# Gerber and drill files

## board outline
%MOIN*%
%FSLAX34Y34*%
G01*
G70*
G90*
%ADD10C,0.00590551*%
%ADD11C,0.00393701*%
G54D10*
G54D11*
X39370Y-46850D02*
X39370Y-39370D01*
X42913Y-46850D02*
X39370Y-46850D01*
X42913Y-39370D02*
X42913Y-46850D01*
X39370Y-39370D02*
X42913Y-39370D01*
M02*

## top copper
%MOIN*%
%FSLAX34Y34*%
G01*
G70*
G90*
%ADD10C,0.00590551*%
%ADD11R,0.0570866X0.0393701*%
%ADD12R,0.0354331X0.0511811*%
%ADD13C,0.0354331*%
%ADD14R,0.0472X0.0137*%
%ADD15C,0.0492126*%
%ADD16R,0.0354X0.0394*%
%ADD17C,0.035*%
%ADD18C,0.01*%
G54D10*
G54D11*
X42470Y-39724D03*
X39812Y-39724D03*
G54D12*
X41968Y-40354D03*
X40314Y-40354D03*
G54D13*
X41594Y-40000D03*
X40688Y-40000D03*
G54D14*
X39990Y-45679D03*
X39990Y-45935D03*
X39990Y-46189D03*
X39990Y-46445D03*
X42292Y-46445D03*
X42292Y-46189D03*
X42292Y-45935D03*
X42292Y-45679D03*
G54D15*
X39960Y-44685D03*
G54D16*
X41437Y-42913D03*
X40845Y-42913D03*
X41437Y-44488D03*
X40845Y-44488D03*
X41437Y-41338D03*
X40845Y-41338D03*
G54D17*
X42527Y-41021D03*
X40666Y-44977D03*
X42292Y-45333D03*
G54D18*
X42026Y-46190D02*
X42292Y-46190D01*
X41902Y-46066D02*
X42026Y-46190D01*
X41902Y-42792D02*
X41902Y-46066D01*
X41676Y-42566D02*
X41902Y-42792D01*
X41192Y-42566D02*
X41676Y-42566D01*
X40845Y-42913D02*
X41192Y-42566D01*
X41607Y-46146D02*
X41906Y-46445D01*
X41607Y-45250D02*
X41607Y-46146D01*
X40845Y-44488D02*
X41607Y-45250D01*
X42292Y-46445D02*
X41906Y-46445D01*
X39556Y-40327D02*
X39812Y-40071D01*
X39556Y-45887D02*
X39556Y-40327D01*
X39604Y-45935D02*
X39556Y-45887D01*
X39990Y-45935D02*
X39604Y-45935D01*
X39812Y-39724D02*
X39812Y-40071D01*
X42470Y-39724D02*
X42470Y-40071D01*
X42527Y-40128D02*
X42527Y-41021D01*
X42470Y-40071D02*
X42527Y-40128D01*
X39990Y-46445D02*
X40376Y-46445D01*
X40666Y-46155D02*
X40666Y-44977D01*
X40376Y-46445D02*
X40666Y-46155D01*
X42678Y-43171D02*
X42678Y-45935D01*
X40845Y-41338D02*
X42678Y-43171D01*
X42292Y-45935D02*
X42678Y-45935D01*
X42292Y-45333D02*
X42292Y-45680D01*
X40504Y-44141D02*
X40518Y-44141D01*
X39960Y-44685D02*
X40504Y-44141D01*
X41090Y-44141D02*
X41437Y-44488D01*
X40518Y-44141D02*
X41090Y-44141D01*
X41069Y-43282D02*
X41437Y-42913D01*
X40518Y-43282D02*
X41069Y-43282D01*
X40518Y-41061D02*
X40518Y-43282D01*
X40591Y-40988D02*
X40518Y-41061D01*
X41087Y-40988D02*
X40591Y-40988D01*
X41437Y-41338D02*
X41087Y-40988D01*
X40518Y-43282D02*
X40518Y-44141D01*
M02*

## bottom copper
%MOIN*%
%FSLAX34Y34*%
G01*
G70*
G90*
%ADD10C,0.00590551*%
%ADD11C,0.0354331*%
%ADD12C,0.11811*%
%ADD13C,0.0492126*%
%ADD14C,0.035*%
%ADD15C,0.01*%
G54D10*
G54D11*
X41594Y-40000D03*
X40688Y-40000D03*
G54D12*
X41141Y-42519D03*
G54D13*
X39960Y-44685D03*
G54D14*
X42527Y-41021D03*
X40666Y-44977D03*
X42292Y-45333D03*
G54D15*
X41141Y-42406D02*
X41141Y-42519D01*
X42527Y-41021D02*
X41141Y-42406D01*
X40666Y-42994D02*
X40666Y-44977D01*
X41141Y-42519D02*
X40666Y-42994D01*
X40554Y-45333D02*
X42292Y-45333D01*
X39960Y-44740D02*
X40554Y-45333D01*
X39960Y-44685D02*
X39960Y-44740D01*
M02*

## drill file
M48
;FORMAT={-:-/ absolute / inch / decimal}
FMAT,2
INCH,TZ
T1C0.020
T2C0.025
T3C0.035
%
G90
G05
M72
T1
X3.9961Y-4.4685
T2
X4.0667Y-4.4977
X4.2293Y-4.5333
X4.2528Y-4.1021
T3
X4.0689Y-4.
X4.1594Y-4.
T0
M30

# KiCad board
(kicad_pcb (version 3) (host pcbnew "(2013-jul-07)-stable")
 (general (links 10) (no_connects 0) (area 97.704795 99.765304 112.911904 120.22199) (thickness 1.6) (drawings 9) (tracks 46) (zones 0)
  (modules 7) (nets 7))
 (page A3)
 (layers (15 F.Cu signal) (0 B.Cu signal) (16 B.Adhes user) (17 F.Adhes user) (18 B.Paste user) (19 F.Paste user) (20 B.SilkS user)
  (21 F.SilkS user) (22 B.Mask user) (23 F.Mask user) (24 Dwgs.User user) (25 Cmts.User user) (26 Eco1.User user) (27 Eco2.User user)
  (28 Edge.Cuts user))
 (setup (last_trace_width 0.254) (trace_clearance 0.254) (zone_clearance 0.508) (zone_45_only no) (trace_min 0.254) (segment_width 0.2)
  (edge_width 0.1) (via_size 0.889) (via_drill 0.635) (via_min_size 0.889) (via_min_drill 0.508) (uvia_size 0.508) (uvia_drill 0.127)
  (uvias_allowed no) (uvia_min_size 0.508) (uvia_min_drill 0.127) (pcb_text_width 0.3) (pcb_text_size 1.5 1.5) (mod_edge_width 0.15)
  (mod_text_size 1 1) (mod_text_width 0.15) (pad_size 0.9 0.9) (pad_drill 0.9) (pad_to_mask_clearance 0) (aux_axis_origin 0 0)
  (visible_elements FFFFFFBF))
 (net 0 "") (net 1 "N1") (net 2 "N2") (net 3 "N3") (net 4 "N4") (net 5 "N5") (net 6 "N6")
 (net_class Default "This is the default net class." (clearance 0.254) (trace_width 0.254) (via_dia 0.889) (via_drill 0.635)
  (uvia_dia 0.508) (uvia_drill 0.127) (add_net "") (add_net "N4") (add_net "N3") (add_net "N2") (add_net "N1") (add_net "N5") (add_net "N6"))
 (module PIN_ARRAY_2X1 (layer F.Cu) (at 104.5 101.6 180)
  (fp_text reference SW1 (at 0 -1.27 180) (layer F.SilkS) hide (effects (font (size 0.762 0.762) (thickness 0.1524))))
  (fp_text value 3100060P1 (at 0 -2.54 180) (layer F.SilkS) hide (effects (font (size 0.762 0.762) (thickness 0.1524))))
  (pad 1 smd rect (at -3.375 0.7 180) (size 1.45 1) (layers F.Cu F.Paste F.Mask) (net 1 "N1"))
  (pad 2 smd rect (at 3.375 0.7 180) (size 1.45 1) (layers F.Cu F.Paste F.Mask) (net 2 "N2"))
  (pad 3 smd rect (at -2.1 -0.9 180) (size 0.9 1.3) (layers F.Cu F.Paste F.Mask))
  (pad 4 smd rect (at 2.1 -0.9 180) (size 0.9 1.3) (layers F.Cu F.Paste F.Mask))
  (pad "" thru_hole circle (at -1.15 0 180) (size 0.9 0.9) (drill 0.9) (layers *.Cu *.Mask F.SilkS))
  (pad "" thru_hole circle (at 1.15 0 180) (size 0.9 0.9) (drill 0.9) (layers *.Cu *.Mask F.SilkS)))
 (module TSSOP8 (layer F.Cu) (at 104.5 117)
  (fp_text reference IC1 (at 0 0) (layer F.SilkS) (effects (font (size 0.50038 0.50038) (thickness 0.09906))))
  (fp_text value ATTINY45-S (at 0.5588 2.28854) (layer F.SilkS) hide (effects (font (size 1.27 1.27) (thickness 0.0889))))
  (pad 1 smd rect (at -2.92354 -0.97282) (size 1.19888 0.34798) (layers F.Cu F.Paste F.Mask))
  (pad 2 smd rect (at -2.92354 -0.32258) (size 1.19888 0.34798) (layers F.Cu F.Paste F.Mask) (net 2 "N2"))
  (pad 3 smd rect (at -2.92354 0.32258) (size 1.19888 0.34798) (layers F.Cu F.Paste F.Mask))
  (pad 4 smd rect (at -2.92354 0.97282) (size 1.19888 0.34798) (layers F.Cu F.Paste F.Mask) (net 1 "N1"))
  (pad 5 smd rect (at 2.92354 0.97282) (size 1.19888 0.34798) (layers F.Cu F.Paste F.Mask) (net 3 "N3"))
  (pad 6 smd rect (at 2.92354 0.32258) (size 1.19888 0.34798) (layers F.Cu F.Paste F.Mask) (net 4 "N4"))
  (pad 7 smd rect (at 2.92354 -0.32258) (size 1.19888 0.34798) (layers F.Cu F.Paste F.Mask) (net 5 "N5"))
  (pad 8 smd rect (at 2.92354 -0.97282) (size 1.19888 0.34798) (layers F.Cu F.Paste F.Mask) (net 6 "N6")))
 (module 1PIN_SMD (layer B.Cu) (at 104.5 108)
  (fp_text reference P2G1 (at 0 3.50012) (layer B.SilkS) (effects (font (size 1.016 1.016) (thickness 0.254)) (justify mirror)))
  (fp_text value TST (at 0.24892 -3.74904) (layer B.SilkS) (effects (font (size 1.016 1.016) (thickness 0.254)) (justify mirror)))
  (pad 1 smd circle (at 0 0) (size 3 3) (layers B.Cu B.Paste B.SilkS B.Mask) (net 1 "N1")))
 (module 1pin (layer F.Cu) (at 101.5 113.5)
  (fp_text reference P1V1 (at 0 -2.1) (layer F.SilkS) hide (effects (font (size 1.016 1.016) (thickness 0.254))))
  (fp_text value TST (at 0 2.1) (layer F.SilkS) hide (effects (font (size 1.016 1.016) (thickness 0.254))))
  (pad 1 thru_hole circle (at 0 0) (size 1.25 1.25) (drill 0.5) (layers *.Cu *.Mask F.SilkS) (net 6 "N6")))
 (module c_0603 (layer F.Cu) (at 104.5 109)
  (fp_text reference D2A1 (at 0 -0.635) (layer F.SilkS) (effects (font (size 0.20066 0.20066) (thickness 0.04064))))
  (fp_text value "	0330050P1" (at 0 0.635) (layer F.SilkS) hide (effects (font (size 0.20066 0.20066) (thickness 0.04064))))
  (pad 1 smd rect (at 0.75184 0) (size 0.89916 1.00076) (layers F.Cu F.Paste F.Mask) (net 6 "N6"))
  (pad 2 smd rect (at -0.75184 0) (size 0.89916 1.00076) (layers F.Cu F.Paste F.Mask) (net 4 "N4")))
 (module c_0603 (layer F.Cu) (at 104.5 113)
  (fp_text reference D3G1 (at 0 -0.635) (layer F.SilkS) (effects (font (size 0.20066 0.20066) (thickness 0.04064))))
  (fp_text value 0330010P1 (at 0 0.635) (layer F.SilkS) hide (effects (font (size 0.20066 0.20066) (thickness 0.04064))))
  (pad 1 smd rect (at 0.75184 0) (size 0.89916 1.00076) (layers F.Cu F.Paste F.Mask) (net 6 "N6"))
  (pad 2 smd rect (at -0.75184 0) (size 0.89916 1.00076) (layers F.Cu F.Paste F.Mask) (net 3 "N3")))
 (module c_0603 (layer F.Cu) (at 104.5 105)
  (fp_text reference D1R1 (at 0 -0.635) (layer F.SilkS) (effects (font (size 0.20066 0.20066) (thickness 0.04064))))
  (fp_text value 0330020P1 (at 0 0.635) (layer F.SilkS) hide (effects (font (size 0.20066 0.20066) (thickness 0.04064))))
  (pad 1 smd rect (at 0.75184 0) (size 0.89916 1.00076) (layers F.Cu F.Paste F.Mask) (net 6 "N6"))
  (pad 2 smd rect (at -0.75184 0) (size 0.89916 1.00076) (layers F.Cu F.Paste F.Mask) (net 5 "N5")))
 (gr_line (start 100 119) (end 100 100) (angle 90) (layer Edge.Cuts) (width 0.1))
 (gr_line (start 109 119) (end 100 119) (angle 90) (layer Edge.Cuts) (width 0.1))
 (gr_line (start 109 100) (end 109 119) (angle 90) (layer Edge.Cuts) (width 0.1))
 (gr_line (start 100 100) (end 109 100) (angle 90) (layer Edge.Cuts) (width 0.1))
 (segment (start 106.7483 117.3226) (end 107.4235 117.3226) (width 0.254) (layer F.Cu) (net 4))
 (segment (start 106.4335 117.0078) (end 106.7483 117.3226) (width 0.254) (layer F.Cu) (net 4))
 (segment (start 106.4335 108.6924) (end 106.4335 117.0078) (width 0.254) (layer F.Cu) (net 4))
 (segment (start 105.8593 108.1182) (end 106.4335 108.6924) (width 0.254) (layer F.Cu) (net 4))
 (segment (start 104.63 108.1182) (end 105.8593 108.1182) (width 0.254) (layer F.Cu) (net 4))
 (segment (start 103.7482 109) (end 104.63 108.1182) (width 0.254) (layer F.Cu) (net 4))
 (segment (start 105.6833 117.2133) (end 106.4428 117.9728) (width 0.254) (layer F.Cu) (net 3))
 (segment (start 105.6833 114.9351) (end 105.6833 117.2133) (width 0.254) (layer F.Cu) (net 3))
 (segment (start 103.7482 113) (end 105.6833 114.9351) (width 0.254) (layer F.Cu) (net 3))
 (segment (start 107.4235 117.9728) (end 106.4428 117.9728) (width 0.254) (layer F.Cu) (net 3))
 (segment (start 100.4738 102.4325) (end 101.125 101.7813) (width 0.254) (layer F.Cu) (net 2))
 (segment (start 100.4738 116.5554) (end 100.4738 102.4325) (width 0.254) (layer F.Cu) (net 2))
 (segment (start 100.5958 116.6774) (end 100.4738 116.5554) (width 0.254) (layer F.Cu) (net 2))
 (segment (start 101.5765 116.6774) (end 100.5958 116.6774) (width 0.254) (layer F.Cu) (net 2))
 (segment (start 101.125 100.9) (end 101.125 101.7813) (width 0.254) (layer F.Cu) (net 2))
 (via (at 108.02 104.1936) (size 0.889) (layers F.Cu B.Cu) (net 1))
 (via (at 103.294 114.2421) (size 0.889) (layers F.Cu B.Cu) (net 1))
 (segment (start 107.875 100.9) (end 107.875 101.7813) (width 0.254) (layer F.Cu) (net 1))
 (segment (start 108.02 101.9263) (end 108.02 104.1936) (width 0.254) (layer F.Cu) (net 1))
 (segment (start 107.875 101.7813) (end 108.02 101.9263) (width 0.254) (layer F.Cu) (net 1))
 (segment (start 101.5765 117.9728) (end 102.5572 117.9728) (width 0.254) (layer F.Cu) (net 1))
 (segment (start 104.5 107.7136) (end 104.5 108) (width 0.254) (layer B.Cu) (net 1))
 (segment (start 108.02 104.1936) (end 104.5 107.7136) (width 0.254) (layer B.Cu) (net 1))
 (segment (start 103.294 109.206) (end 103.294 114.2421) (width 0.254) (layer B.Cu) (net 1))
 (segment (start 104.5 108) (end 103.294 109.206) (width 0.254) (layer B.Cu) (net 1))
 (segment (start 103.294 117.236) (end 103.294 114.2421) (width 0.254) (layer F.Cu) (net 1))
 (segment (start 102.5572 117.9728) (end 103.294 117.236) (width 0.254) (layer F.Cu) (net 1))
 (segment (start 108.4042 109.656) (end 108.4042 116.6774) (width 0.254) (layer F.Cu) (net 5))
 (segment (start 103.7482 105) (end 108.4042 109.656) (width 0.254) (layer F.Cu) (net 5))
 (segment (start 107.4235 116.6774) (end 108.4042 116.6774) (width 0.254) (layer F.Cu) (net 5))
 (via (at 107.4235 115.147) (size 0.889) (layers F.Cu B.Cu) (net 6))
 (segment (start 103.0072 115.147) (end 107.4235 115.147) (width 0.254) (layer B.Cu) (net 6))
 (segment (start 101.5 113.6398) (end 103.0072 115.147) (width 0.254) (layer B.Cu) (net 6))
 (segment (start 101.5 113.5) (end 101.5 113.6398) (width 0.254) (layer B.Cu) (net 6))
 (segment (start 107.4235 115.147) (end 107.4235 116.0272) (width 0.254) (layer F.Cu) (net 6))
 (segment (start 102.8818 112.1182) (end 102.9172 112.1182) (width 0.254) (layer F.Cu) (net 6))
 (segment (start 101.5 113.5) (end 102.8818 112.1182) (width 0.254) (layer F.Cu) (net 6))
 (segment (start 104.37 112.1182) (end 105.2518 113) (width 0.254) (layer F.Cu) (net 6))
 (segment (start 102.9172 112.1182) (end 104.37 112.1182) (width 0.254) (layer F.Cu) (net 6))
 (segment (start 104.3154 109.9364) (end 105.2518 109) (width 0.254) (layer F.Cu) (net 6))
 (segment (start 102.9172 109.9364) (end 104.3154 109.9364) (width 0.254) (layer F.Cu) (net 6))
 (segment (start 102.9172 104.297) (end 102.9172 109.9364) (width 0.254) (layer F.Cu) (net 6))
 (segment (start 103.1034 104.1108) (end 102.9172 104.297) (width 0.254) (layer F.Cu) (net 6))
 (segment (start 104.3626 104.1108) (end 103.1034 104.1108) (width 0.254) (layer F.Cu) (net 6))
 (segment (start 105.2518 105) (end 104.3626 104.1108) (width 0.254) (layer F.Cu) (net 6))
 (segment (start 102.9172 109.9364) (end 102.9172 112.1182) (width 0.254) (layer F.Cu) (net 6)))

